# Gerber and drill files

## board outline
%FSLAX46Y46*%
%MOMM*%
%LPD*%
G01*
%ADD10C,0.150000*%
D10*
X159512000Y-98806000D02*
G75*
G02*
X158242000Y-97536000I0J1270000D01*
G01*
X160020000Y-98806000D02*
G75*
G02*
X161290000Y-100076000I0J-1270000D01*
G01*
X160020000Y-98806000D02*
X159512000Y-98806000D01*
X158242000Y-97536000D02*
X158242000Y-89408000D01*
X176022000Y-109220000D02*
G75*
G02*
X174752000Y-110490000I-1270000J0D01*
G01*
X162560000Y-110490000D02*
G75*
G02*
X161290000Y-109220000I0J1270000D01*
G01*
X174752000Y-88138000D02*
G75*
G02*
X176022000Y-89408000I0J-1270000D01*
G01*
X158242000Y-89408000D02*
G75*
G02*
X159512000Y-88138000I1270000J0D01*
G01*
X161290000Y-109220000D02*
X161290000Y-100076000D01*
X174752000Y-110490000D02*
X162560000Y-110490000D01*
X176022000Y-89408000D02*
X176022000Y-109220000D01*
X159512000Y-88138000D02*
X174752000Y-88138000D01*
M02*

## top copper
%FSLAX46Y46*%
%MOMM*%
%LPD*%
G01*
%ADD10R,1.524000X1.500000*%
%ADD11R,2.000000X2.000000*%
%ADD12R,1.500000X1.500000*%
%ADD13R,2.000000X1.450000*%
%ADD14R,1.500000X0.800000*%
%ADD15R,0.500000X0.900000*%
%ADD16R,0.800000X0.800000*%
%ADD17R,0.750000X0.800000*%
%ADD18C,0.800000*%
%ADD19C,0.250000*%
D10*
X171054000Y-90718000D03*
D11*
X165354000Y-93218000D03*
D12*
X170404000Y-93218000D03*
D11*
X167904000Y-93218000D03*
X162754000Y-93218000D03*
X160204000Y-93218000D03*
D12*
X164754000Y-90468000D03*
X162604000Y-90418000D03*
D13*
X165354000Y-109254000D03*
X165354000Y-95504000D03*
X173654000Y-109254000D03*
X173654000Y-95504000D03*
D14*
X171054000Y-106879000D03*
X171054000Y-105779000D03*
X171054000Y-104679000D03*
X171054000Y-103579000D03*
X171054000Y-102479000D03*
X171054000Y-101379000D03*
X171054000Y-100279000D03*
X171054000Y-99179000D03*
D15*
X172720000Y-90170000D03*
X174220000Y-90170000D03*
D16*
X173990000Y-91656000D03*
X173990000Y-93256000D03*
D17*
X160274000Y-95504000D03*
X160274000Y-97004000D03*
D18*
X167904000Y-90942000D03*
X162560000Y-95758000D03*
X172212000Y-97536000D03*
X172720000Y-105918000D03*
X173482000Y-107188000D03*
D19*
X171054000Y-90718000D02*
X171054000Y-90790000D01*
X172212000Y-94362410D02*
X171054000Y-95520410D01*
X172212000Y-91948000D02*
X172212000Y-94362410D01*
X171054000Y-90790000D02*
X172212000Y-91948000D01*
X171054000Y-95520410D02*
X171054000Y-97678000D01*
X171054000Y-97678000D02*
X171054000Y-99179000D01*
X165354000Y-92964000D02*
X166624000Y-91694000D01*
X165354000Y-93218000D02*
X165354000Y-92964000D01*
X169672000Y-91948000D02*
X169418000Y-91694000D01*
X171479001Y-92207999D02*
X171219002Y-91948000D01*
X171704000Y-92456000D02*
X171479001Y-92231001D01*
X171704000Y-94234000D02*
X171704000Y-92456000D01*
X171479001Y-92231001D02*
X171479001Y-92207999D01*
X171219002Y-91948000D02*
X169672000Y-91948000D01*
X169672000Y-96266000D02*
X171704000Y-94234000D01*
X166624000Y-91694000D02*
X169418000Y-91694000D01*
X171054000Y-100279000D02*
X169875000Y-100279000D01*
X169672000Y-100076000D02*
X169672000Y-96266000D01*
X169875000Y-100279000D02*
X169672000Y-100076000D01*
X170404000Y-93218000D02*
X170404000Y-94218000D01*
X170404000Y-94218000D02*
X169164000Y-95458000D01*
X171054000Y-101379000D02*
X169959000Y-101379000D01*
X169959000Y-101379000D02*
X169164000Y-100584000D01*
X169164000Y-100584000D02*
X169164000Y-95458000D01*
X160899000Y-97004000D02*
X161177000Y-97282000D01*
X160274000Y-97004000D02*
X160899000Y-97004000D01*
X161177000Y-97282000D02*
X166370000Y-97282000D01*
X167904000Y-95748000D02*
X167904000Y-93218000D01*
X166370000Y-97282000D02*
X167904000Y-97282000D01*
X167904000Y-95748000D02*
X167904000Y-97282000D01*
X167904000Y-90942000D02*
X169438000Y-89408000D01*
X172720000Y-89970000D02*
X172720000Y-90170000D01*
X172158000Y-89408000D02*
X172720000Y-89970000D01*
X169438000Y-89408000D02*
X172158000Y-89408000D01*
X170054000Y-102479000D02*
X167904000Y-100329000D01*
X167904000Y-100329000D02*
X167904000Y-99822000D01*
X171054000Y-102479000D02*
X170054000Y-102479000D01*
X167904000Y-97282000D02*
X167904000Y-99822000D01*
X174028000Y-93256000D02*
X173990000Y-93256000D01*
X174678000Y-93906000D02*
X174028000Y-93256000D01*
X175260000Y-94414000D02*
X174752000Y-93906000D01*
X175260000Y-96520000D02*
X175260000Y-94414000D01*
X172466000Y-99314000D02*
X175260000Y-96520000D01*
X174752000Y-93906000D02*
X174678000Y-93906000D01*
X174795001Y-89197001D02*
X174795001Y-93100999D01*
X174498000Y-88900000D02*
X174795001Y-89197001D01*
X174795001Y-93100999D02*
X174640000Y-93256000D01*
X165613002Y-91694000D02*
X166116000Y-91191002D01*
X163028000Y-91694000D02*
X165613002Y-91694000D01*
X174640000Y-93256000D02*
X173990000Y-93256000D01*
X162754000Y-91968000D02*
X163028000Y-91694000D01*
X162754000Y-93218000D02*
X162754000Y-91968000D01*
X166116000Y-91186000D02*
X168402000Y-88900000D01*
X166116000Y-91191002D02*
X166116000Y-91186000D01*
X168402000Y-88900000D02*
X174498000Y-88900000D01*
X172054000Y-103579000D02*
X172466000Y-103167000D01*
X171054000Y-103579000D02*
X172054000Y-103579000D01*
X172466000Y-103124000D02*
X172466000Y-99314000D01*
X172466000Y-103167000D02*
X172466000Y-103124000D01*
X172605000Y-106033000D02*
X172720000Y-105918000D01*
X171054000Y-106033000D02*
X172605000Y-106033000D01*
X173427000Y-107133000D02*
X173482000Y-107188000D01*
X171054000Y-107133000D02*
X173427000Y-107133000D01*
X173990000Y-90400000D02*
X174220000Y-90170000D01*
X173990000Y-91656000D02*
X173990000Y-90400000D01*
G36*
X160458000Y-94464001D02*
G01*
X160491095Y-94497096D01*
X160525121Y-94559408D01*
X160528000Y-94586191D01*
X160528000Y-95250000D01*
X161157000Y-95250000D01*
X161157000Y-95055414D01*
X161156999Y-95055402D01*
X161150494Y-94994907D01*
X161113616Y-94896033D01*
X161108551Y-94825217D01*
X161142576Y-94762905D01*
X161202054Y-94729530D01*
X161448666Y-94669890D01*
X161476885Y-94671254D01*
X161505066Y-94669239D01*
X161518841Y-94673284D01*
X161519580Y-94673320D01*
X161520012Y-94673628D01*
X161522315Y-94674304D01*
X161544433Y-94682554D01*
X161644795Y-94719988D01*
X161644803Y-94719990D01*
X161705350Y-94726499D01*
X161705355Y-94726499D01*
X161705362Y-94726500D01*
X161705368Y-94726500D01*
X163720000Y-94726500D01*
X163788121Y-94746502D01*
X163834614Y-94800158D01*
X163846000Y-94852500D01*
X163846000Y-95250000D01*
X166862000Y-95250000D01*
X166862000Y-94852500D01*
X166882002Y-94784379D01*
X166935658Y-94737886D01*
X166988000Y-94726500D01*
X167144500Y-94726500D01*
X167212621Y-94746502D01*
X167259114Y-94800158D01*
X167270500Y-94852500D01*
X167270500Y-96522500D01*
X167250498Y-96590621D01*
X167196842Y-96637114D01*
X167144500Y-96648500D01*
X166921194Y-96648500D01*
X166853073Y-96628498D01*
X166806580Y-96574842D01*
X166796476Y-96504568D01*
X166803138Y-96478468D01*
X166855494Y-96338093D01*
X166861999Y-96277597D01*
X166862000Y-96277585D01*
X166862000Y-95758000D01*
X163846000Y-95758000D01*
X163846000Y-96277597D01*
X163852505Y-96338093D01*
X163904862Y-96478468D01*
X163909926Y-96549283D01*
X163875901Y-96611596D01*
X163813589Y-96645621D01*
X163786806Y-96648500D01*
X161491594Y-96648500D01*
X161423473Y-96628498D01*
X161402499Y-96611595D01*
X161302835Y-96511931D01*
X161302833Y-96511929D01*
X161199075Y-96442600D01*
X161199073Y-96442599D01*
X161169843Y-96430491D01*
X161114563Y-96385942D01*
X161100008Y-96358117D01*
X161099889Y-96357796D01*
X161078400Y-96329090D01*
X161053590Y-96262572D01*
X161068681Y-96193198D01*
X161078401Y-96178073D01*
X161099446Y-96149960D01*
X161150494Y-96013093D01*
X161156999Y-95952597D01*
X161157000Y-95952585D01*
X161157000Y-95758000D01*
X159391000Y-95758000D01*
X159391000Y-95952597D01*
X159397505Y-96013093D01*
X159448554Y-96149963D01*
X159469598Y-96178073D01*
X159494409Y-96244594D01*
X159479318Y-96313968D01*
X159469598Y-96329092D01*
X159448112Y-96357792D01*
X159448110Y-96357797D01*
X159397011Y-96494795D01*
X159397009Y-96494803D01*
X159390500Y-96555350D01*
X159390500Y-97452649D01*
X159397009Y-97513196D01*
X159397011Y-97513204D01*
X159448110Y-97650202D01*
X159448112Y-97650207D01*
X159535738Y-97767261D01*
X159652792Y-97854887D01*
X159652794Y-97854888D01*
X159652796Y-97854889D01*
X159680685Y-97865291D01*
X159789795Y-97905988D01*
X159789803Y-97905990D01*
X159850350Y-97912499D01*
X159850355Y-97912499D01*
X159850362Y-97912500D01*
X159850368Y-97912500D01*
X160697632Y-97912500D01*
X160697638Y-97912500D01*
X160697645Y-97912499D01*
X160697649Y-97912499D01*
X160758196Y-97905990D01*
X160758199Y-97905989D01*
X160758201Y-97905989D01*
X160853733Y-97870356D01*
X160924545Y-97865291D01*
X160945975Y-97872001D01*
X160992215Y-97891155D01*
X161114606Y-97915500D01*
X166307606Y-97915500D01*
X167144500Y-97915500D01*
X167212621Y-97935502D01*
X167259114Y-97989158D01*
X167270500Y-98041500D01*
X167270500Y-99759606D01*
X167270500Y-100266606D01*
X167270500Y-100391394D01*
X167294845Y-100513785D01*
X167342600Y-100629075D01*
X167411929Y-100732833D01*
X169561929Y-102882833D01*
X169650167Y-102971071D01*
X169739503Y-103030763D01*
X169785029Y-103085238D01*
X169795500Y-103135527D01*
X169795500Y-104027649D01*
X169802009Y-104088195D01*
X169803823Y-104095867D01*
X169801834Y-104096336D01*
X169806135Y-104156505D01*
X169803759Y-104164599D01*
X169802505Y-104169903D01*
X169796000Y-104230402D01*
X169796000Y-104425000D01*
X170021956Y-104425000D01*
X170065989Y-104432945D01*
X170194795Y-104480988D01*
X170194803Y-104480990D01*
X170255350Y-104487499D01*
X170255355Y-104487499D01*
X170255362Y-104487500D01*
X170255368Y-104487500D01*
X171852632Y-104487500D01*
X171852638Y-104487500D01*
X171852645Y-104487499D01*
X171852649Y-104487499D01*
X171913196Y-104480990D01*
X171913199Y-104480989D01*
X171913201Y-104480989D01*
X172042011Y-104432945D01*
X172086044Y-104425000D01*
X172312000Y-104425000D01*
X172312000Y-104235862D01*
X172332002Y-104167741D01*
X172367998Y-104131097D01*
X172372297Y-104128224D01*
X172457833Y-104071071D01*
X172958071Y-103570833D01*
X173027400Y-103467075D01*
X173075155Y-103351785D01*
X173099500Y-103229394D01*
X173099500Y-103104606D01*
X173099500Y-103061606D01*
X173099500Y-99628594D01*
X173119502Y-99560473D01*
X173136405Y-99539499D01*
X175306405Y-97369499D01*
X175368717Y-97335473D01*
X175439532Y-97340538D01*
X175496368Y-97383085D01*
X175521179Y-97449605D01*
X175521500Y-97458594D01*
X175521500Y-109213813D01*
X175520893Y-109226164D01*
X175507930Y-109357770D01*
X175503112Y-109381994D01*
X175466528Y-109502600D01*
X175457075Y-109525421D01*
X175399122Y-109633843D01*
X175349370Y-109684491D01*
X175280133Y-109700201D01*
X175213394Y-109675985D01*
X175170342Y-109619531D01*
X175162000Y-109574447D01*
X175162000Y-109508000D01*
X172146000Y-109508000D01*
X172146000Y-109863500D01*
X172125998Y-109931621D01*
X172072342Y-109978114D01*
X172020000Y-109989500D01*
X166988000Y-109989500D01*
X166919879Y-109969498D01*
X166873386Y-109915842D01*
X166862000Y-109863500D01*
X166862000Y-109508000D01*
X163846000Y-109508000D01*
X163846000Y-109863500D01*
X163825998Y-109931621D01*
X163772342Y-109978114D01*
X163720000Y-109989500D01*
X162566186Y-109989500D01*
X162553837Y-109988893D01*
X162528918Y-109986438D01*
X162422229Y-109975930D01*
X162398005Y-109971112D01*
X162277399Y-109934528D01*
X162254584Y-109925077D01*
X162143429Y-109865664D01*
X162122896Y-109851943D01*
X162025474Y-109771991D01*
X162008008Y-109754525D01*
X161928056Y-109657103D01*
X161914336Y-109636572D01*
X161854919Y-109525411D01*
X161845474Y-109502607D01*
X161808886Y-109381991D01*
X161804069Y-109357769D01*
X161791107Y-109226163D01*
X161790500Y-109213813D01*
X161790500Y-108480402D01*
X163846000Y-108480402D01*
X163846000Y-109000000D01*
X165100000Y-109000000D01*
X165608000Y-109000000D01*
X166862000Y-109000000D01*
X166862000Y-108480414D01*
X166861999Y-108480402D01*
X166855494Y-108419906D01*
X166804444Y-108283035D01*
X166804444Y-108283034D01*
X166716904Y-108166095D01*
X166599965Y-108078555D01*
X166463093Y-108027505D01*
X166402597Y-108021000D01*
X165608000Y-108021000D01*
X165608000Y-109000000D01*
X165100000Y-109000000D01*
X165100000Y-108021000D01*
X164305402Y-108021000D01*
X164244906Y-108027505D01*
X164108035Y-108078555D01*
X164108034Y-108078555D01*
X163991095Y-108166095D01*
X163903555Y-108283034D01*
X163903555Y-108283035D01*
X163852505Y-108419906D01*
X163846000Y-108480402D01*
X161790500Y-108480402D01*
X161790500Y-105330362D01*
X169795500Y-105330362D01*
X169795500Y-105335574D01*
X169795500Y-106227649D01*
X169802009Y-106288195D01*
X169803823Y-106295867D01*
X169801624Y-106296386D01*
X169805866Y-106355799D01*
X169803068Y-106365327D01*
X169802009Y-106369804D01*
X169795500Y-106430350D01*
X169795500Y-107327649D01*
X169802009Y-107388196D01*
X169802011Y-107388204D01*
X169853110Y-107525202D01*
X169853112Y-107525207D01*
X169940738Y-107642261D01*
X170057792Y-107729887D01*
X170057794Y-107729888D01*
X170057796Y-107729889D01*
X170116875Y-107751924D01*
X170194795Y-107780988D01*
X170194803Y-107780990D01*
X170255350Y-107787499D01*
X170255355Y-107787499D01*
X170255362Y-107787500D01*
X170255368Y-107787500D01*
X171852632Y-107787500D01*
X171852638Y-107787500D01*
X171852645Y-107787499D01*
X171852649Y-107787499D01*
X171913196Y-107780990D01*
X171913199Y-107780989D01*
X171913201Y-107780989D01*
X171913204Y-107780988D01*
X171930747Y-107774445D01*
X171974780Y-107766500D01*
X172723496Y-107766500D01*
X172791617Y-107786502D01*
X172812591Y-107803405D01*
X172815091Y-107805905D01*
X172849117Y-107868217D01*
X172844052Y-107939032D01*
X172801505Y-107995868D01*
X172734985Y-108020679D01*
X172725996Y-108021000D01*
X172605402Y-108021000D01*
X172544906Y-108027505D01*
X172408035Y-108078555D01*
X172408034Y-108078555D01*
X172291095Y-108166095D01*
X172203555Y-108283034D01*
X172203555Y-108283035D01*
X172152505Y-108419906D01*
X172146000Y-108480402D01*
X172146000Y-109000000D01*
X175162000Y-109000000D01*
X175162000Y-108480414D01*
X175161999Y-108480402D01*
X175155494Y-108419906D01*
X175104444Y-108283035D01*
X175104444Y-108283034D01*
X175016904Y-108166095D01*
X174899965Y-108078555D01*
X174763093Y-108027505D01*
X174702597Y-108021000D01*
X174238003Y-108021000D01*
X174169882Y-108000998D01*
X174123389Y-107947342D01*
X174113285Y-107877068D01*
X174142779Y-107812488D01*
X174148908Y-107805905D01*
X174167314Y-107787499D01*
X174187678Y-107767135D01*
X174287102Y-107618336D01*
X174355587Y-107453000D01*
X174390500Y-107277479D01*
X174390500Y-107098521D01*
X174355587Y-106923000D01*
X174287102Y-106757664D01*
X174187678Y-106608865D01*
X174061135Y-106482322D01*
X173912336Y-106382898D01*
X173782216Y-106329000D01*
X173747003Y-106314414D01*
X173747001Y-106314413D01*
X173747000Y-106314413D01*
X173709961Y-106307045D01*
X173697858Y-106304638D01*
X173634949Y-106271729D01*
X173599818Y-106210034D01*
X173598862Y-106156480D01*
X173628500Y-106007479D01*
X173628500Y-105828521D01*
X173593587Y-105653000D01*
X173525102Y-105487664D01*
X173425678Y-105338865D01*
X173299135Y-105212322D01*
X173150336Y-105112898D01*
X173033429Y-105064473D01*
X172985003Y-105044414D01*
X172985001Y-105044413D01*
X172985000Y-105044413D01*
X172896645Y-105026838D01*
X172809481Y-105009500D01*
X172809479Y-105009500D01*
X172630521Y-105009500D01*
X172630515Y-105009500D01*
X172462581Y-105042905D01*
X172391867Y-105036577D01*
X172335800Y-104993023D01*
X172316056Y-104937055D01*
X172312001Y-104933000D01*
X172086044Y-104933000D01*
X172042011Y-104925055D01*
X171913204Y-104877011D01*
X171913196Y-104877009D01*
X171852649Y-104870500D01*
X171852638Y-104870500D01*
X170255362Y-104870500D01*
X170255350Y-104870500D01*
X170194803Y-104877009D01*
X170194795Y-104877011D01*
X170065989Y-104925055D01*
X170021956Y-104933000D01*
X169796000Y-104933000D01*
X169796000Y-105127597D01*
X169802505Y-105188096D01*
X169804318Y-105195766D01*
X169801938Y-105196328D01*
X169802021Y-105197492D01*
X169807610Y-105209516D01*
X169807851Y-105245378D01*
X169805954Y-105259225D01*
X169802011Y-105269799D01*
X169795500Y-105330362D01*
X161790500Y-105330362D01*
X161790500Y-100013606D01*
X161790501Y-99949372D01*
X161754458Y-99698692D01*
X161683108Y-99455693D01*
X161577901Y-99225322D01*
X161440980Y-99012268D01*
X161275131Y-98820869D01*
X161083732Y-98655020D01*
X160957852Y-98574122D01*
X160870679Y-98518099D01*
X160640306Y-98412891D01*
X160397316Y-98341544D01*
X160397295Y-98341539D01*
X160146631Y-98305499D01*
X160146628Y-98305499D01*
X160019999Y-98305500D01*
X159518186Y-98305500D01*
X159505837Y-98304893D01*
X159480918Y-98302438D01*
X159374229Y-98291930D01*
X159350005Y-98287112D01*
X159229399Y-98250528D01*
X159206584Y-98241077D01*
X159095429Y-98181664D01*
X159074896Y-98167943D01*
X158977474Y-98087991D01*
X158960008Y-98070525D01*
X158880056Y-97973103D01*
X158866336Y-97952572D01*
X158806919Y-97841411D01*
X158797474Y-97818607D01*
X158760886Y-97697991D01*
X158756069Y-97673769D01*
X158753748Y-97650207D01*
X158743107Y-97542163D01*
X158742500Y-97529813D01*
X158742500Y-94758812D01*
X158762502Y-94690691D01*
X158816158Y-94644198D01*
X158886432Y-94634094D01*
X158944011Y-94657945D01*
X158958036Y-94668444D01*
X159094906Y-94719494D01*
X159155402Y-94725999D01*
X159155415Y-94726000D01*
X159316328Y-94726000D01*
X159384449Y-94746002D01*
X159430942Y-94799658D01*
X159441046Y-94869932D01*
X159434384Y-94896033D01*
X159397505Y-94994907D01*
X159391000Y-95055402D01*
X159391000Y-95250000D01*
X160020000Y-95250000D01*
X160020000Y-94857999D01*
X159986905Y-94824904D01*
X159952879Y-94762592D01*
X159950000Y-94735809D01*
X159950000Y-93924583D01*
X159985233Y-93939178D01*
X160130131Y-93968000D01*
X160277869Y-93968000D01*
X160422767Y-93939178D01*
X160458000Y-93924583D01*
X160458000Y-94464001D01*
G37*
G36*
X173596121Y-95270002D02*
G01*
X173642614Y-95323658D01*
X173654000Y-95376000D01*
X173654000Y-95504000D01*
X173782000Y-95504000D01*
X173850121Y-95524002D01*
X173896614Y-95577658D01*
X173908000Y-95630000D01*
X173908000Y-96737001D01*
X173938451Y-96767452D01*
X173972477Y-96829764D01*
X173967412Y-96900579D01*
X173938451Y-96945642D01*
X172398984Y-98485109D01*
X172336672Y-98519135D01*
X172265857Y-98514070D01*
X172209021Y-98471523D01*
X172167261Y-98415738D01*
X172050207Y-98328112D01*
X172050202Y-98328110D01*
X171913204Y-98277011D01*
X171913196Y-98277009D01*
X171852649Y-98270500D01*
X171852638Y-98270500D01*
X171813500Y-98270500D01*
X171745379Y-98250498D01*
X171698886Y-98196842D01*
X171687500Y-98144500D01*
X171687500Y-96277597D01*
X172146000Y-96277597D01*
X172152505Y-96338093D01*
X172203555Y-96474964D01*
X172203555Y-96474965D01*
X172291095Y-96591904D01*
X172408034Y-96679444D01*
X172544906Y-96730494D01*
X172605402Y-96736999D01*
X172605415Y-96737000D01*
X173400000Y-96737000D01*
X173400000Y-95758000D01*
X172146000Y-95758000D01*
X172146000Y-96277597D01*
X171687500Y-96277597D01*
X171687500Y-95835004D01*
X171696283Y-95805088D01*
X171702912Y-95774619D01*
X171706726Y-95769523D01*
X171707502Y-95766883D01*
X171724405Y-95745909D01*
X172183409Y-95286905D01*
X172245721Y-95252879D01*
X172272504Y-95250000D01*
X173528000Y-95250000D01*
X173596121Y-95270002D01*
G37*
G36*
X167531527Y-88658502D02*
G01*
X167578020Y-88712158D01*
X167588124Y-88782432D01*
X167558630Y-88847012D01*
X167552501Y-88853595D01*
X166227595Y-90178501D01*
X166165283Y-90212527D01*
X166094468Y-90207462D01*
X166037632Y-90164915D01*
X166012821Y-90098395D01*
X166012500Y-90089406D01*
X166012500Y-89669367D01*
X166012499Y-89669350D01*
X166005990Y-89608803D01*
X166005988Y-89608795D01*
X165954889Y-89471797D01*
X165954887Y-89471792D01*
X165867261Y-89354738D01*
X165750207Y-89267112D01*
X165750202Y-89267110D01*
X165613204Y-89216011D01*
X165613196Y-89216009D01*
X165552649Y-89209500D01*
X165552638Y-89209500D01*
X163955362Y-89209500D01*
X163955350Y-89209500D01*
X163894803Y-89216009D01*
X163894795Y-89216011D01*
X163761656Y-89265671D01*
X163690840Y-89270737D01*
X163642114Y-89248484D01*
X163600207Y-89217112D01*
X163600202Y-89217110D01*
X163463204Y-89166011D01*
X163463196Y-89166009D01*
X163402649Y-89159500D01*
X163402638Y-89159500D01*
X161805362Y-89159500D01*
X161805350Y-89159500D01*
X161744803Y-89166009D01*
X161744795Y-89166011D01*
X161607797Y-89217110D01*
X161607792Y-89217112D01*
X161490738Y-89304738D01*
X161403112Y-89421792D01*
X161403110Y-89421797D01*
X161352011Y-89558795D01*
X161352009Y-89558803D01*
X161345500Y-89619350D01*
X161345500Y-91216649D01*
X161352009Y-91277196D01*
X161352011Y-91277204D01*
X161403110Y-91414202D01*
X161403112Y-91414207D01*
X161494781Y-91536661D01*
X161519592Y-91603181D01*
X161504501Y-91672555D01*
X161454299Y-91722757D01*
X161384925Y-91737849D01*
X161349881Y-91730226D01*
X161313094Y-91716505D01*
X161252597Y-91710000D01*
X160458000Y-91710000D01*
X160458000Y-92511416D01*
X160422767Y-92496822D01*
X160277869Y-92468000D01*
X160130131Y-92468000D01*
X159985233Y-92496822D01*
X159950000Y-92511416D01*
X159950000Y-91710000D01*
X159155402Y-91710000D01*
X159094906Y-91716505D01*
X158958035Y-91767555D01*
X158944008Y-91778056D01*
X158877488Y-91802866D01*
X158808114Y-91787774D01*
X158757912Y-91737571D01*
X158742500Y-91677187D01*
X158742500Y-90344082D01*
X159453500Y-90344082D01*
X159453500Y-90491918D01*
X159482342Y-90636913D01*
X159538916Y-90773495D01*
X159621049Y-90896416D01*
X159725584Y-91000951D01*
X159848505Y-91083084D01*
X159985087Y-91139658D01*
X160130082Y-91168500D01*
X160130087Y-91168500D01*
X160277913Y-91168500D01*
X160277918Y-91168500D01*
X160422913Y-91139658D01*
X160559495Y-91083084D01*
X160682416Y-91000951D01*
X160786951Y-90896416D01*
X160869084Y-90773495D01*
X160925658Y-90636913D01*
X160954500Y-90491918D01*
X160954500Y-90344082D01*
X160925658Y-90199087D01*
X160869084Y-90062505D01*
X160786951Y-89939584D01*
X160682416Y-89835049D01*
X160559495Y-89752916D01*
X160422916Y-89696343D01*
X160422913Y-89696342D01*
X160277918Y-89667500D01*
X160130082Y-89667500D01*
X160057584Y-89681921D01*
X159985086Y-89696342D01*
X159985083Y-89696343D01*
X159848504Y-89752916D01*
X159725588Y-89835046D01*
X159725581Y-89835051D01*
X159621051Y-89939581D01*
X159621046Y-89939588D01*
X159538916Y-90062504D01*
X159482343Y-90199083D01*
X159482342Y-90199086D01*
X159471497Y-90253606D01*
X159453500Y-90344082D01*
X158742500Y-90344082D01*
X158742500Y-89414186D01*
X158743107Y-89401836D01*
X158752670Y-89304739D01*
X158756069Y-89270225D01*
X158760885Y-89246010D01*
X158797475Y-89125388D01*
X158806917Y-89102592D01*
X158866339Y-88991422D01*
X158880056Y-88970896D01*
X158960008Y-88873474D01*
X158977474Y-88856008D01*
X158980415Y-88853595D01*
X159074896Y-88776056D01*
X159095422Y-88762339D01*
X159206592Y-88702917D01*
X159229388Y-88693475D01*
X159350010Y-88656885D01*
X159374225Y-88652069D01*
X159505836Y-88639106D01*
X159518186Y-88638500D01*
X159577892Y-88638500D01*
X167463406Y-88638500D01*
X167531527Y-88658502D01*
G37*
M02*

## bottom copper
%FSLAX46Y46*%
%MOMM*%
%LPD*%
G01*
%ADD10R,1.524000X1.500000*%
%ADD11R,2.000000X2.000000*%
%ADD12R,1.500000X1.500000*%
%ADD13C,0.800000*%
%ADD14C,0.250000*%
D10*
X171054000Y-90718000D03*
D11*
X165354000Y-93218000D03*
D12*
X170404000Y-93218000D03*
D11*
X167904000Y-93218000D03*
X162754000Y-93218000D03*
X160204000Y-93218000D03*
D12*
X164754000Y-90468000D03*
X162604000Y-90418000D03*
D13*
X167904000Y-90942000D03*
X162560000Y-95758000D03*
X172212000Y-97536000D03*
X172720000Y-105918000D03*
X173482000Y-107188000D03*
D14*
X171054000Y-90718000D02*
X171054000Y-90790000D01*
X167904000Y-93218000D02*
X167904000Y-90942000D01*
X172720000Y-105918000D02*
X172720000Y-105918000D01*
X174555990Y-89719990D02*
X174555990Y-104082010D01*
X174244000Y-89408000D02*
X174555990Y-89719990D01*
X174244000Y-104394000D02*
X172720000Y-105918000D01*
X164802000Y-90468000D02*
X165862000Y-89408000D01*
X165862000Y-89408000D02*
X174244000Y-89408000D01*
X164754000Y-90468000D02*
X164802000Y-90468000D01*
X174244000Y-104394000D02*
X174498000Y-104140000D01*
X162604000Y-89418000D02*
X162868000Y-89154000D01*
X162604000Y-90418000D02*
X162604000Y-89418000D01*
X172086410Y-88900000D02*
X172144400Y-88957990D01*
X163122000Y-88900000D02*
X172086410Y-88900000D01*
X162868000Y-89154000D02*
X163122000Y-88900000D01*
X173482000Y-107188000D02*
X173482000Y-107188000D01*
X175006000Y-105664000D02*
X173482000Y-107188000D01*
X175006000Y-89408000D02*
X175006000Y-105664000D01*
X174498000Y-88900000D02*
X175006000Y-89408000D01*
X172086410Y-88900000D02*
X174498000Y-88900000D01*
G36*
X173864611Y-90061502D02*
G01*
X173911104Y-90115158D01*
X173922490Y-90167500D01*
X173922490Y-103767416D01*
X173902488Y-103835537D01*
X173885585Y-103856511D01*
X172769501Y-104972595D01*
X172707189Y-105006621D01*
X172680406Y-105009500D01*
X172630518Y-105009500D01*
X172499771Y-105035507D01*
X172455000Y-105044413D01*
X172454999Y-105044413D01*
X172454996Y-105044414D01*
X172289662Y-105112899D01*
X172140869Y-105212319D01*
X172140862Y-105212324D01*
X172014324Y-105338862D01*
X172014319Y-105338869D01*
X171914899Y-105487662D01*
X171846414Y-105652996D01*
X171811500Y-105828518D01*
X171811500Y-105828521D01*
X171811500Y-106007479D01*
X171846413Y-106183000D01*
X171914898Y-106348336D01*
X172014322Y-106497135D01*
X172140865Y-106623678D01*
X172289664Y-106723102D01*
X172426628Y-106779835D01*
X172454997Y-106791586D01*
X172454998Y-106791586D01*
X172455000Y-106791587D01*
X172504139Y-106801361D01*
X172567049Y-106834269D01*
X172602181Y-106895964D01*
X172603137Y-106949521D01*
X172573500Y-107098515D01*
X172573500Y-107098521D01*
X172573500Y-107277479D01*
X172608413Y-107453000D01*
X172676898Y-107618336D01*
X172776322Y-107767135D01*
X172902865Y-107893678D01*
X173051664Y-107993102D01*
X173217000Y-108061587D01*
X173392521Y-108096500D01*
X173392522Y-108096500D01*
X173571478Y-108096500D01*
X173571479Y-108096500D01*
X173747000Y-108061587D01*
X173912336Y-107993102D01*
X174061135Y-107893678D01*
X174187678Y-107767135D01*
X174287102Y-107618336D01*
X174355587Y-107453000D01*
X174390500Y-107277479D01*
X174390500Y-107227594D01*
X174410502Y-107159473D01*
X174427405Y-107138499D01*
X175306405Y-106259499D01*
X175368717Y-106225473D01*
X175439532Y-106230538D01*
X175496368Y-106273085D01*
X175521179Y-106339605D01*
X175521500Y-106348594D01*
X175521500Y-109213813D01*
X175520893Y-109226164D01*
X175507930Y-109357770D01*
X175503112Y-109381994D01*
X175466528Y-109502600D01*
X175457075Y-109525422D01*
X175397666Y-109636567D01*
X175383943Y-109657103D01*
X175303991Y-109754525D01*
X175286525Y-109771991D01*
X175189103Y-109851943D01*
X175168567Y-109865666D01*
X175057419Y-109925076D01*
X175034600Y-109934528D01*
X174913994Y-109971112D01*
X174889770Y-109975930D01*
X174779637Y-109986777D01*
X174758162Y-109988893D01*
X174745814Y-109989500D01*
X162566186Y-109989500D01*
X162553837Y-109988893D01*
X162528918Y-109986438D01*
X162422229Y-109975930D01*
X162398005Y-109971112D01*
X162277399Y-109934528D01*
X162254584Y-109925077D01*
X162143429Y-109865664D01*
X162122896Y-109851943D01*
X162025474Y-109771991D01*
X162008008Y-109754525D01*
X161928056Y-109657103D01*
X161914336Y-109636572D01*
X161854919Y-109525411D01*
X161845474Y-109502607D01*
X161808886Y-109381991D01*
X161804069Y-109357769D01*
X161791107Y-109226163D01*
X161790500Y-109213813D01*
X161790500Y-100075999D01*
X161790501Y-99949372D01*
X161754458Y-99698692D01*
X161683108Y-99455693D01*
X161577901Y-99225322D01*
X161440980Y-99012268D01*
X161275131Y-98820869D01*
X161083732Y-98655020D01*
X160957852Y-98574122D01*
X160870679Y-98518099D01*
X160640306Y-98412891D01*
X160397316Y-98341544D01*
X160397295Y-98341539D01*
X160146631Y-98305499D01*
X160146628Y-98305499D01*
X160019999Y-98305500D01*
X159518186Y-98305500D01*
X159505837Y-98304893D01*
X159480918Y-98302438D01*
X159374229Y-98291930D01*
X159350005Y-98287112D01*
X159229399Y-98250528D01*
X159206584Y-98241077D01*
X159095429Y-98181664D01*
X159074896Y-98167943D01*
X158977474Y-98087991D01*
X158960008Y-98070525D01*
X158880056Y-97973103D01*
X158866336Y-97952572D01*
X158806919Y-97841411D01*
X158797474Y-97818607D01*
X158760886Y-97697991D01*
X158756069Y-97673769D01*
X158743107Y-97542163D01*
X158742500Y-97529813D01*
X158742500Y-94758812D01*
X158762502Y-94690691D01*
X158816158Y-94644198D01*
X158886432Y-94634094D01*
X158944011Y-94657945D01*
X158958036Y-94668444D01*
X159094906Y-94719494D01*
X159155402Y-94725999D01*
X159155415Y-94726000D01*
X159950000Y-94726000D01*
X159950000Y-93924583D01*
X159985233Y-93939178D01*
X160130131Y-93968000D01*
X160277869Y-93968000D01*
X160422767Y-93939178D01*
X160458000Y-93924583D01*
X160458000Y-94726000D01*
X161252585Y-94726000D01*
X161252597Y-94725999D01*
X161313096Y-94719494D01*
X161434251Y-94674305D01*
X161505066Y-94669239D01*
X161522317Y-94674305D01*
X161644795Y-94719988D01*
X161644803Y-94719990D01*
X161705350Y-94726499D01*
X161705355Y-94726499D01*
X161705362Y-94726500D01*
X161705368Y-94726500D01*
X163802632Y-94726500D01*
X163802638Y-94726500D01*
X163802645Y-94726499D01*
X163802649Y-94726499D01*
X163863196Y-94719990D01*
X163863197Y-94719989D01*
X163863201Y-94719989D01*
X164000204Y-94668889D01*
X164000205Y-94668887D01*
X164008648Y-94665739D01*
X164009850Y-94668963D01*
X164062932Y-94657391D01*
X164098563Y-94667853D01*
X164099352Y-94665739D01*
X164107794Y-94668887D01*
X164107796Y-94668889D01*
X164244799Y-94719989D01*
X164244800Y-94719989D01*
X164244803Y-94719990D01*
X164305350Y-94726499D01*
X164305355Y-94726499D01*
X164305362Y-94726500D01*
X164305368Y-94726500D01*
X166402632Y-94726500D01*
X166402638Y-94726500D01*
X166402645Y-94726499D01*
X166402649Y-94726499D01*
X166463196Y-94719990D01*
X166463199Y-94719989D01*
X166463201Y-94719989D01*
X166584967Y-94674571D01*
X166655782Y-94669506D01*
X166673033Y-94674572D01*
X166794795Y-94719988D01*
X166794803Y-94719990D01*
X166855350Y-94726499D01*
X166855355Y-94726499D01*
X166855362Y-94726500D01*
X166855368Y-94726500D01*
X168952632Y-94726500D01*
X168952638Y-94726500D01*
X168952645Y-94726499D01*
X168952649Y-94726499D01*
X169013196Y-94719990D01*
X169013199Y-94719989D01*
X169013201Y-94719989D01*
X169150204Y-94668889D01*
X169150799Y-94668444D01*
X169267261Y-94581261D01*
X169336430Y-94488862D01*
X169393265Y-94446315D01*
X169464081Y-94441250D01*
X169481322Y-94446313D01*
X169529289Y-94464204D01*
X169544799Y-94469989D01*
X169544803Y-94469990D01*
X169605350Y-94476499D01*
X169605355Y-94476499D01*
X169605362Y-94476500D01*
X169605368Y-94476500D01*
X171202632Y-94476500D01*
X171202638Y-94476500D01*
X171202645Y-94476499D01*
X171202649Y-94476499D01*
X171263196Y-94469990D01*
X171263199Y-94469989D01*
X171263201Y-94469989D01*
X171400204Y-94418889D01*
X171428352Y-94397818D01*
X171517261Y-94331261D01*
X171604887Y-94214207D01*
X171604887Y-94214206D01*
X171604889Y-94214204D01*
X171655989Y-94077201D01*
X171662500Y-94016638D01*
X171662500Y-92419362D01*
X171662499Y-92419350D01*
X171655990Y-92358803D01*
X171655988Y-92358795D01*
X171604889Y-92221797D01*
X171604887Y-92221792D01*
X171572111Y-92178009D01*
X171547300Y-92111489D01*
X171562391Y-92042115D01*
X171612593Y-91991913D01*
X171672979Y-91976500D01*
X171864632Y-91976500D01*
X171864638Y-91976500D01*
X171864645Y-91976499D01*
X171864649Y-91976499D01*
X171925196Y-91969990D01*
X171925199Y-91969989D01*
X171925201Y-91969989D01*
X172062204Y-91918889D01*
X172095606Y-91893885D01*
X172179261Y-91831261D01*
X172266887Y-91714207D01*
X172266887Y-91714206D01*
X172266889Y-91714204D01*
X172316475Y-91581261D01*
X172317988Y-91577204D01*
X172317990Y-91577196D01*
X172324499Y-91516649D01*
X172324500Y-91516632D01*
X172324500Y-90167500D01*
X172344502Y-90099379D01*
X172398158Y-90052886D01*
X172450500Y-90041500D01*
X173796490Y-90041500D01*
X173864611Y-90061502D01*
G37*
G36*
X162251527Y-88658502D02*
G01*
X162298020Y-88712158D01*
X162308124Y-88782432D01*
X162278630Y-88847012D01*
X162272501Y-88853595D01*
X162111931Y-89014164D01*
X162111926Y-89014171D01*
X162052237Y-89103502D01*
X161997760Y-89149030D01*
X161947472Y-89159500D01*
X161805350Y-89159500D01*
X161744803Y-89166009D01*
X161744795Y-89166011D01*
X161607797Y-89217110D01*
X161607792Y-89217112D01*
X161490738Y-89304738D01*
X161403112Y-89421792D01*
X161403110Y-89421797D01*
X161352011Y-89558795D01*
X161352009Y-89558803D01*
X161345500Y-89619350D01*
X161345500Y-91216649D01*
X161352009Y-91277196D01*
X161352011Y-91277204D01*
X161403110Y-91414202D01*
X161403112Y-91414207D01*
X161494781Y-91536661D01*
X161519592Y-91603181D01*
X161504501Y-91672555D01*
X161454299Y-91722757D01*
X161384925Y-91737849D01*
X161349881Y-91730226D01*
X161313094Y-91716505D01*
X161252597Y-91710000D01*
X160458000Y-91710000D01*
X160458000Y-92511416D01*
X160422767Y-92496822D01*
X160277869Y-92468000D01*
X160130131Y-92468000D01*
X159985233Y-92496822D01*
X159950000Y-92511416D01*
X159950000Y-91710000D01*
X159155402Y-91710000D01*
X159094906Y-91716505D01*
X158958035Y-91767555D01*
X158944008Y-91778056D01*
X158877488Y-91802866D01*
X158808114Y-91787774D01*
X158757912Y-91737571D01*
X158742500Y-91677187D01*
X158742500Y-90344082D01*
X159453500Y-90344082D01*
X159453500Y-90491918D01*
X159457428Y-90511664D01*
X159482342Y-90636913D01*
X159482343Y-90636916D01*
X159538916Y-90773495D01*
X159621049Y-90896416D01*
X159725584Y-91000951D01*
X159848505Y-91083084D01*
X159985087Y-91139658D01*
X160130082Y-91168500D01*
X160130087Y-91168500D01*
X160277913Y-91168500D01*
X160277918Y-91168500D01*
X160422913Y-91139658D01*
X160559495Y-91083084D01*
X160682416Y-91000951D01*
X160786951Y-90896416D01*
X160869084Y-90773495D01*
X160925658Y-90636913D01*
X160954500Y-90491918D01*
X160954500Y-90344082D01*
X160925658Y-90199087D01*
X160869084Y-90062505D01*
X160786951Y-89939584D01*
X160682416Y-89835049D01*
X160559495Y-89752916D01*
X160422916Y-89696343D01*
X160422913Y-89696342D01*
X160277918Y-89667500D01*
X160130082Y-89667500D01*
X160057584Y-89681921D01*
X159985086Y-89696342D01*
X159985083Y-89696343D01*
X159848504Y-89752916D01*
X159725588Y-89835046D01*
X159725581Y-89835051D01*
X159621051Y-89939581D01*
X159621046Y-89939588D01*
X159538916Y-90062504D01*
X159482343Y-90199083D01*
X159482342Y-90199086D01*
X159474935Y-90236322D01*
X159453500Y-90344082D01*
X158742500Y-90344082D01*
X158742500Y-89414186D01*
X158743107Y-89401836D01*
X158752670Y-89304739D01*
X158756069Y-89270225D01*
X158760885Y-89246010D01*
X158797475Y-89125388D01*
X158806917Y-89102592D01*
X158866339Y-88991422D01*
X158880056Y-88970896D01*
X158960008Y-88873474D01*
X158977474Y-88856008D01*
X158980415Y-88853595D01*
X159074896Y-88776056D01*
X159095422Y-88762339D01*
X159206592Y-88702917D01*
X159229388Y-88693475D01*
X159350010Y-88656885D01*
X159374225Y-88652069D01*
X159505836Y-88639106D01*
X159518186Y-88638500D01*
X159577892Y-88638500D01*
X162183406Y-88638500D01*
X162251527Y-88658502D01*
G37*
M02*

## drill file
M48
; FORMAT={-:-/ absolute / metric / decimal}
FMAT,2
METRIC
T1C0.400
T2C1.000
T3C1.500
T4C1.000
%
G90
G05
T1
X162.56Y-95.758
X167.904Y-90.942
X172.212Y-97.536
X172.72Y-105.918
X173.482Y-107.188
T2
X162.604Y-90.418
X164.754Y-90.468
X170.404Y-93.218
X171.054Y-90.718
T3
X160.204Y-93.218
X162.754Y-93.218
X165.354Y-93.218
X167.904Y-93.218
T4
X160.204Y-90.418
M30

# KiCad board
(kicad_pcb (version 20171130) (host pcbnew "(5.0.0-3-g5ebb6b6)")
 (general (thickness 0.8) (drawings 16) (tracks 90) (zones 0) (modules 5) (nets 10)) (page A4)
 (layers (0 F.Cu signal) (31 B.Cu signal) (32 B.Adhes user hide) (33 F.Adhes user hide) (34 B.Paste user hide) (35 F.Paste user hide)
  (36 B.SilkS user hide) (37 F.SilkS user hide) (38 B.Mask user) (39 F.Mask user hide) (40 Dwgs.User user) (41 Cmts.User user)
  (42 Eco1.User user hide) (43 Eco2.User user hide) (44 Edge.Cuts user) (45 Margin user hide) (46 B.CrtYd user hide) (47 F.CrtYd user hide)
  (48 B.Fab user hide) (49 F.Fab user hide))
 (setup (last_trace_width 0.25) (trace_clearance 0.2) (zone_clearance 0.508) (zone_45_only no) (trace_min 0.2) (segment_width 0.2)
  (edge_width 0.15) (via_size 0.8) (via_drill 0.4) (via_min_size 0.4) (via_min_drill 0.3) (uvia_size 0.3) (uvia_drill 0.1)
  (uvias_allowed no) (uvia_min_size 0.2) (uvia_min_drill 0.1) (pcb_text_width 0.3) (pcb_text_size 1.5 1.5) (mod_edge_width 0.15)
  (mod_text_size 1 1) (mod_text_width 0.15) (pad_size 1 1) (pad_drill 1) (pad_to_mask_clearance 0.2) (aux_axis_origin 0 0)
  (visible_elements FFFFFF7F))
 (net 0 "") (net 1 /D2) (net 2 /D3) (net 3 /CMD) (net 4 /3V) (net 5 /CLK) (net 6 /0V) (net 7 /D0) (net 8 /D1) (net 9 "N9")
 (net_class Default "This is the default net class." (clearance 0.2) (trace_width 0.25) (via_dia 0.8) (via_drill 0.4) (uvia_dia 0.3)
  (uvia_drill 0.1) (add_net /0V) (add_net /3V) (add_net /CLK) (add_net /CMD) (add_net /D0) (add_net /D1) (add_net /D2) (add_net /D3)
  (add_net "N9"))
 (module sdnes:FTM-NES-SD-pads (layer F.Cu) (at 165.354 93.218)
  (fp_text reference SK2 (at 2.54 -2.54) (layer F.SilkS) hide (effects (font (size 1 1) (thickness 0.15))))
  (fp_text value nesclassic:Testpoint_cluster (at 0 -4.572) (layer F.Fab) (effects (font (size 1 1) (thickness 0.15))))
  (pad 1 thru_hole rect (at 5.7 -2.5 270) (size 1.5 1.524) (drill 1) (layers *.Cu *.Mask) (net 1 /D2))
  (pad 2 thru_hole rect (at 0 0) (size 2 2) (drill 1.5) (layers *.Cu *.Mask) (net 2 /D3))
  (pad 3 thru_hole rect (at 5.05 0) (size 1.5 1.5) (drill 1) (layers *.Cu *.Mask) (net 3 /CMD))
  (pad 4 thru_hole rect (at 2.55 0) (size 2 2) (drill 1.5) (layers *.Cu *.Mask) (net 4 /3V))
  (pad 5 thru_hole rect (at -2.6 0) (size 2 2) (drill 1.5) (layers *.Cu *.Mask) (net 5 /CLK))
  (pad 6 thru_hole rect (at -5.15 0) (size 2 2) (drill 1.5) (layers *.Cu *.Mask) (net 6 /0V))
  (pad 7 thru_hole rect (at -0.6 -2.75) (size 1.5 1.5) (drill 1) (layers *.Cu *.Mask) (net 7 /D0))
  (pad 8 thru_hole rect (at -2.75 -2.8) (size 1.5 1.5) (drill 1) (layers *.Cu *.Mask) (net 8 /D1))
  (pad "" np_thru_hole circle (at -5.15 -2.8) (size 1 1) (drill 1) (layers *.Cu *.Mask)))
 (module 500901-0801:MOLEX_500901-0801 (layer F.Cu) (at 171.054 102.379 270)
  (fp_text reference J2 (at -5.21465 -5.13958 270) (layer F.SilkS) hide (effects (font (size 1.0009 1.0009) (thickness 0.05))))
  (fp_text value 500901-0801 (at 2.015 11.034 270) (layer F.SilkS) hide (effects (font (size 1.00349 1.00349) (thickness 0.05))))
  (pad SH4 smd rect (at 6.875 5.7) (size 2 1.45) (layers F.Cu F.Paste F.Mask) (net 6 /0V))
  (pad SH3 smd rect (at -6.875 5.7) (size 2 1.45) (layers F.Cu F.Paste F.Mask) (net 6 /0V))
  (pad SH2 smd rect (at 6.875 -2.6) (size 2 1.45) (layers F.Cu F.Paste F.Mask) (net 6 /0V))
  (pad SH1 smd rect (at -6.875 -2.6) (size 2 1.45) (layers F.Cu F.Paste F.Mask) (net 6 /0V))
  (pad 8 smd rect (at 4.5 0) (size 1.5 0.8) (layers F.Cu F.Paste F.Mask) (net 8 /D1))
  (pad 7 smd rect (at 3.4 0) (size 1.5 0.8) (layers F.Cu F.Paste F.Mask) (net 7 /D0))
  (pad 6 smd rect (at 2.3 0) (size 1.5 0.8) (layers F.Cu F.Paste F.Mask) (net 6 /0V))
  (pad 5 smd rect (at 1.2 0) (size 1.5 0.8) (layers F.Cu F.Paste F.Mask) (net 5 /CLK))
  (pad 4 smd rect (at 0.1 0) (size 1.5 0.8) (layers F.Cu F.Paste F.Mask) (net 4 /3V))
  (pad 3 smd rect (at -1 0) (size 1.5 0.8) (layers F.Cu F.Paste F.Mask) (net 3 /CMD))
  (pad 2 smd rect (at -2.1 0) (size 1.5 0.8) (layers F.Cu F.Paste F.Mask) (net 2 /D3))
  (pad 1 smd rect (at -3.2 0) (size 1.5 0.8) (layers F.Cu F.Paste F.Mask) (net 1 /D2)))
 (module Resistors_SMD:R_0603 (layer F.Cu) (at 173.47 90.17)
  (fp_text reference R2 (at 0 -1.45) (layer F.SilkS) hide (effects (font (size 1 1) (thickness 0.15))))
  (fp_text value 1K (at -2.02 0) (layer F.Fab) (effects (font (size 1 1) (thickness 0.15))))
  (pad 1 smd rect (at -0.75 0) (size 0.5 0.9) (layers F.Cu F.Paste F.Mask) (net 4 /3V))
  (pad 2 smd rect (at 0.75 0) (size 0.5 0.9) (layers F.Cu F.Paste F.Mask) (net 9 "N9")))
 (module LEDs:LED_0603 (layer F.Cu) (at 173.99 92.456 90)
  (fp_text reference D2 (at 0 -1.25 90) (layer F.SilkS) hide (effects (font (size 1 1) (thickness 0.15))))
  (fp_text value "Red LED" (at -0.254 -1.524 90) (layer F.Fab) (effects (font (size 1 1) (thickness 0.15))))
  (pad 2 smd rect (at 0.8 0 270) (size 0.8 0.8) (layers F.Cu F.Paste F.Mask) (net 9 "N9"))
  (pad 1 smd rect (at -0.8 0 270) (size 0.8 0.8) (layers F.Cu F.Paste F.Mask) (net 5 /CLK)))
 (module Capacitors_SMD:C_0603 (layer F.Cu) (at 160.274 96.254 90)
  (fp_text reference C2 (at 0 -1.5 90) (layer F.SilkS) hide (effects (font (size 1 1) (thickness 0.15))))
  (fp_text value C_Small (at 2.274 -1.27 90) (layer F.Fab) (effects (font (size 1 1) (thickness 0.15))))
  (pad 2 smd rect (at 0.75 0 90) (size 0.8 0.75) (layers F.Cu F.Paste F.Mask) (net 6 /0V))
  (pad 1 smd rect (at -0.75 0 90) (size 0.8 0.75) (layers F.Cu F.Paste F.Mask) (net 4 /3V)))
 (gr_arc (start 159.512 97.536) (end 158.242 97.536) (angle -90) (layer Edge.Cuts) (width 0.15))
 (gr_arc (start 160.02 100.076) (end 161.29 100.076) (angle -90) (layer Edge.Cuts) (width 0.15))
 (gr_line (start 160.02 98.806) (end 159.512 98.806) (layer Edge.Cuts) (width 0.15))
 (gr_line (start 158.242 97.536) (end 158.242 89.408) (layer Edge.Cuts) (width 0.15))
 (gr_arc (start 174.752 109.22) (end 174.752 110.49) (angle -90) (layer Edge.Cuts) (width 0.15))
 (gr_arc (start 162.56 109.22) (end 161.29 109.22) (angle -90) (layer Edge.Cuts) (width 0.15))
 (gr_arc (start 174.752 89.408) (end 176.022 89.408) (angle -90) (layer Edge.Cuts) (width 0.15))
 (gr_arc (start 159.512 89.408) (end 159.512 88.138) (angle -90) (layer Edge.Cuts) (width 0.15))
 (gr_line (start 161.29 109.22) (end 161.29 100.076) (layer Edge.Cuts) (width 0.15))
 (gr_line (start 174.752 110.49) (end 162.56 110.49) (layer Edge.Cuts) (width 0.15))
 (gr_line (start 176.022 89.408) (end 176.022 109.22) (layer Edge.Cuts) (width 0.15))
 (gr_line (start 159.512 88.138) (end 174.752 88.138) (layer Edge.Cuts) (width 0.15))
 (segment (start 171.054 90.718) (end 171.054 90.79) (width 0.25) (layer B.Cu) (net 1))
 (segment (start 171.054 90.718) (end 171.054 90.79) (width 0.25) (layer F.Cu) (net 1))
 (segment (start 172.212 94.36241) (end 171.054 95.52041) (width 0.25) (layer F.Cu) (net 1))
 (segment (start 172.212 91.948) (end 172.212 94.36241) (width 0.25) (layer F.Cu) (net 1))
 (segment (start 171.054 90.79) (end 172.212 91.948) (width 0.25) (layer F.Cu) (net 1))
 (segment (start 171.054 95.52041) (end 171.054 97.678) (width 0.25) (layer F.Cu) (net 1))
 (segment (start 171.054 97.678) (end 171.054 99.179) (width 0.25) (layer F.Cu) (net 1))
 (segment (start 165.354 92.964) (end 166.624 91.694) (width 0.25) (layer F.Cu) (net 2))
 (segment (start 165.354 93.218) (end 165.354 92.964) (width 0.25) (layer F.Cu) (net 2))
 (segment (start 169.672 91.948) (end 169.418 91.694) (width 0.25) (layer F.Cu) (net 2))
 (segment (start 171.479001 92.207999) (end 171.219002 91.948) (width 0.25) (layer F.Cu) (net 2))
 (segment (start 171.704 92.456) (end 171.479001 92.231001) (width 0.25) (layer F.Cu) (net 2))
 (segment (start 171.704 94.234) (end 171.704 92.456) (width 0.25) (layer F.Cu) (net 2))
 (segment (start 171.479001 92.231001) (end 171.479001 92.207999) (width 0.25) (layer F.Cu) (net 2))
 (segment (start 171.219002 91.948) (end 169.672 91.948) (width 0.25) (layer F.Cu) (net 2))
 (segment (start 169.672 96.266) (end 171.704 94.234) (width 0.25) (layer F.Cu) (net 2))
 (segment (start 166.624 91.694) (end 169.418 91.694) (width 0.25) (layer F.Cu) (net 2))
 (segment (start 171.054 100.279) (end 169.875 100.279) (width 0.25) (layer F.Cu) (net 2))
 (segment (start 169.672 100.076) (end 169.672 96.266) (width 0.25) (layer F.Cu) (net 2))
 (segment (start 169.875 100.279) (end 169.672 100.076) (width 0.25) (layer F.Cu) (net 2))
 (segment (start 170.404 93.218) (end 170.404 94.218) (width 0.25) (layer F.Cu) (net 3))
 (segment (start 170.404 94.218) (end 169.164 95.458) (width 0.25) (layer F.Cu) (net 3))
 (segment (start 171.054 101.379) (end 169.959 101.379) (width 0.25) (layer F.Cu) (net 3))
 (segment (start 169.959 101.379) (end 169.164 100.584) (width 0.25) (layer F.Cu) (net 3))
 (segment (start 169.164 100.584) (end 169.164 95.458) (width 0.25) (layer F.Cu) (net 3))
 (segment (start 160.899 97.004) (end 161.177 97.282) (width 0.25) (layer F.Cu) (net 4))
 (segment (start 160.274 97.004) (end 160.899 97.004) (width 0.25) (layer F.Cu) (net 4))
 (segment (start 161.177 97.282) (end 166.37 97.282) (width 0.25) (layer F.Cu) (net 4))
 (segment (start 167.904 95.748) (end 167.904 93.218) (width 0.25) (layer F.Cu) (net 4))
 (segment (start 166.37 97.282) (end 167.904 97.282) (width 0.25) (layer F.Cu) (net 4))
 (segment (start 167.904 95.748) (end 167.904 97.282) (width 0.25) (layer F.Cu) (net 4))
 (segment (start 167.904 93.218) (end 167.904 90.942) (width 0.25) (layer B.Cu) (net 4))
 (via (at 167.904 90.942) (size 0.8) (drill 0.4) (layers F.Cu B.Cu) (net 4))
 (segment (start 167.904 90.942) (end 169.438 89.408) (width 0.25) (layer F.Cu) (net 4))
 (segment (start 172.72 89.97) (end 172.72 90.17) (width 0.25) (layer F.Cu) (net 4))
 (segment (start 172.158 89.408) (end 172.72 89.97) (width 0.25) (layer F.Cu) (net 4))
 (segment (start 169.438 89.408) (end 172.158 89.408) (width 0.25) (layer F.Cu) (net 4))
 (segment (start 170.054 102.479) (end 167.904 100.329) (width 0.25) (layer F.Cu) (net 4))
 (segment (start 167.904 100.329) (end 167.904 99.822) (width 0.25) (layer F.Cu) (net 4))
 (segment (start 171.054 102.479) (end 170.054 102.479) (width 0.25) (layer F.Cu) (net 4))
 (segment (start 167.904 97.282) (end 167.904 99.822) (width 0.25) (layer F.Cu) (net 4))
 (segment (start 174.028 93.256) (end 173.99 93.256) (width 0.25) (layer F.Cu) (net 5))
 (segment (start 174.678 93.906) (end 174.028 93.256) (width 0.25) (layer F.Cu) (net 5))
 (segment (start 175.26 94.414) (end 174.752 93.906) (width 0.25) (layer F.Cu) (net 5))
 (segment (start 175.26 96.52) (end 175.26 94.414) (width 0.25) (layer F.Cu) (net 5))
 (segment (start 172.466 99.314) (end 175.26 96.52) (width 0.25) (layer F.Cu) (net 5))
 (segment (start 174.752 93.906) (end 174.678 93.906) (width 0.25) (layer F.Cu) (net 5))
 (segment (start 174.795001 89.197001) (end 174.795001 93.100999) (width 0.25) (layer F.Cu) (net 5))
 (segment (start 174.498 88.9) (end 174.795001 89.197001) (width 0.25) (layer F.Cu) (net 5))
 (segment (start 174.795001 93.100999) (end 174.64 93.256) (width 0.25) (layer F.Cu) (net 5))
 (segment (start 165.613002 91.694) (end 166.116 91.191002) (width 0.25) (layer F.Cu) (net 5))
 (segment (start 163.028 91.694) (end 165.613002 91.694) (width 0.25) (layer F.Cu) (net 5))
 (segment (start 174.64 93.256) (end 173.99 93.256) (width 0.25) (layer F.Cu) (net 5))
 (segment (start 162.754 91.968) (end 163.028 91.694) (width 0.25) (layer F.Cu) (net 5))
 (segment (start 162.754 93.218) (end 162.754 91.968) (width 0.25) (layer F.Cu) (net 5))
 (segment (start 166.116 91.186) (end 168.402 88.9) (width 0.25) (layer F.Cu) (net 5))
 (segment (start 166.116 91.191002) (end 166.116 91.186) (width 0.25) (layer F.Cu) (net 5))
 (segment (start 168.402 88.9) (end 174.498 88.9) (width 0.25) (layer F.Cu) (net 5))
 (segment (start 172.054 103.579) (end 172.466 103.167) (width 0.25) (layer F.Cu) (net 5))
 (segment (start 171.054 103.579) (end 172.054 103.579) (width 0.25) (layer F.Cu) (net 5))
 (segment (start 172.466 103.124) (end 172.466 99.314) (width 0.25) (layer F.Cu) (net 5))
 (segment (start 172.466 103.167) (end 172.466 103.124) (width 0.25) (layer F.Cu) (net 5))
 (via (at 162.56 95.758) (size 0.8) (drill 0.4) (layers F.Cu B.Cu) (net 6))
 (via (at 172.212 97.536) (size 0.8) (drill 0.4) (layers F.Cu B.Cu) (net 6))
 (segment (start 172.72 105.918) (end 172.72 105.918) (width 0.25) (layer B.Cu) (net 7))
 (via (at 172.72 105.918) (size 0.8) (drill 0.4) (layers F.Cu B.Cu) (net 7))
 (segment (start 172.605 106.033) (end 172.72 105.918) (width 0.25) (layer F.Cu) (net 7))
 (segment (start 171.054 106.033) (end 172.605 106.033) (width 0.25) (layer F.Cu) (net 7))
 (segment (start 174.55599 89.71999) (end 174.55599 104.08201) (width 0.25) (layer B.Cu) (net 7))
 (segment (start 174.244 89.408) (end 174.55599 89.71999) (width 0.25) (layer B.Cu) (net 7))
 (segment (start 174.244 104.394) (end 172.72 105.918) (width 0.25) (layer B.Cu) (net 7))
 (segment (start 164.802 90.468) (end 165.862 89.408) (width 0.25) (layer B.Cu) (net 7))
 (segment (start 165.862 89.408) (end 174.244 89.408) (width 0.25) (layer B.Cu) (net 7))
 (segment (start 164.754 90.468) (end 164.802 90.468) (width 0.25) (layer B.Cu) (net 7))
 (segment (start 174.244 104.394) (end 174.498 104.14) (width 0.25) (layer B.Cu) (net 7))
 (segment (start 162.604 89.418) (end 162.868 89.154) (width 0.25) (layer B.Cu) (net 8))
 (segment (start 162.604 90.418) (end 162.604 89.418) (width 0.25) (layer B.Cu) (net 8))
 (segment (start 172.08641 88.9) (end 172.1444 88.95799) (width 0.25) (layer B.Cu) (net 8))
 (segment (start 163.122 88.9) (end 172.08641 88.9) (width 0.25) (layer B.Cu) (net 8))
 (segment (start 162.868 89.154) (end 163.122 88.9) (width 0.25) (layer B.Cu) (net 8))
 (segment (start 173.482 107.188) (end 173.482 107.188) (width 0.25) (layer B.Cu) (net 8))
 (via (at 173.482 107.188) (size 0.8) (drill 0.4) (layers F.Cu B.Cu) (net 8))
 (segment (start 173.427 107.133) (end 173.482 107.188) (width 0.25) (layer F.Cu) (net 8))
 (segment (start 171.054 107.133) (end 173.427 107.133) (width 0.25) (layer F.Cu) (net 8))
 (segment (start 175.006 105.664) (end 173.482 107.188) (width 0.25) (layer B.Cu) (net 8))
 (segment (start 175.006 89.408) (end 175.006 105.664) (width 0.25) (layer B.Cu) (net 8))
 (segment (start 174.498 88.9) (end 175.006 89.408) (width 0.25) (layer B.Cu) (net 8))
 (segment (start 172.08641 88.9) (end 174.498 88.9) (width 0.25) (layer B.Cu) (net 8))
 (segment (start 173.99 90.4) (end 174.22 90.17) (width 0.25) (layer F.Cu) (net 9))
 (segment (start 173.99 91.656) (end 173.99 90.4) (width 0.25) (layer F.Cu) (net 9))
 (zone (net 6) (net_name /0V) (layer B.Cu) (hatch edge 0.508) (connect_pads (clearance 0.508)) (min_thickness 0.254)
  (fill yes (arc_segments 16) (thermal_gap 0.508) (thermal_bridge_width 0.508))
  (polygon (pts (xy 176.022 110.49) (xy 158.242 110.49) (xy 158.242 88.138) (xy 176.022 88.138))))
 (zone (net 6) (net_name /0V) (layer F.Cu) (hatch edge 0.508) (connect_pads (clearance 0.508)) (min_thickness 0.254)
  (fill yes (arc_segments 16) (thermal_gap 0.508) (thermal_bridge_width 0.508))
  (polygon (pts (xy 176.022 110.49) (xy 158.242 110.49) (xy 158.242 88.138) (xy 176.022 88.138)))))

